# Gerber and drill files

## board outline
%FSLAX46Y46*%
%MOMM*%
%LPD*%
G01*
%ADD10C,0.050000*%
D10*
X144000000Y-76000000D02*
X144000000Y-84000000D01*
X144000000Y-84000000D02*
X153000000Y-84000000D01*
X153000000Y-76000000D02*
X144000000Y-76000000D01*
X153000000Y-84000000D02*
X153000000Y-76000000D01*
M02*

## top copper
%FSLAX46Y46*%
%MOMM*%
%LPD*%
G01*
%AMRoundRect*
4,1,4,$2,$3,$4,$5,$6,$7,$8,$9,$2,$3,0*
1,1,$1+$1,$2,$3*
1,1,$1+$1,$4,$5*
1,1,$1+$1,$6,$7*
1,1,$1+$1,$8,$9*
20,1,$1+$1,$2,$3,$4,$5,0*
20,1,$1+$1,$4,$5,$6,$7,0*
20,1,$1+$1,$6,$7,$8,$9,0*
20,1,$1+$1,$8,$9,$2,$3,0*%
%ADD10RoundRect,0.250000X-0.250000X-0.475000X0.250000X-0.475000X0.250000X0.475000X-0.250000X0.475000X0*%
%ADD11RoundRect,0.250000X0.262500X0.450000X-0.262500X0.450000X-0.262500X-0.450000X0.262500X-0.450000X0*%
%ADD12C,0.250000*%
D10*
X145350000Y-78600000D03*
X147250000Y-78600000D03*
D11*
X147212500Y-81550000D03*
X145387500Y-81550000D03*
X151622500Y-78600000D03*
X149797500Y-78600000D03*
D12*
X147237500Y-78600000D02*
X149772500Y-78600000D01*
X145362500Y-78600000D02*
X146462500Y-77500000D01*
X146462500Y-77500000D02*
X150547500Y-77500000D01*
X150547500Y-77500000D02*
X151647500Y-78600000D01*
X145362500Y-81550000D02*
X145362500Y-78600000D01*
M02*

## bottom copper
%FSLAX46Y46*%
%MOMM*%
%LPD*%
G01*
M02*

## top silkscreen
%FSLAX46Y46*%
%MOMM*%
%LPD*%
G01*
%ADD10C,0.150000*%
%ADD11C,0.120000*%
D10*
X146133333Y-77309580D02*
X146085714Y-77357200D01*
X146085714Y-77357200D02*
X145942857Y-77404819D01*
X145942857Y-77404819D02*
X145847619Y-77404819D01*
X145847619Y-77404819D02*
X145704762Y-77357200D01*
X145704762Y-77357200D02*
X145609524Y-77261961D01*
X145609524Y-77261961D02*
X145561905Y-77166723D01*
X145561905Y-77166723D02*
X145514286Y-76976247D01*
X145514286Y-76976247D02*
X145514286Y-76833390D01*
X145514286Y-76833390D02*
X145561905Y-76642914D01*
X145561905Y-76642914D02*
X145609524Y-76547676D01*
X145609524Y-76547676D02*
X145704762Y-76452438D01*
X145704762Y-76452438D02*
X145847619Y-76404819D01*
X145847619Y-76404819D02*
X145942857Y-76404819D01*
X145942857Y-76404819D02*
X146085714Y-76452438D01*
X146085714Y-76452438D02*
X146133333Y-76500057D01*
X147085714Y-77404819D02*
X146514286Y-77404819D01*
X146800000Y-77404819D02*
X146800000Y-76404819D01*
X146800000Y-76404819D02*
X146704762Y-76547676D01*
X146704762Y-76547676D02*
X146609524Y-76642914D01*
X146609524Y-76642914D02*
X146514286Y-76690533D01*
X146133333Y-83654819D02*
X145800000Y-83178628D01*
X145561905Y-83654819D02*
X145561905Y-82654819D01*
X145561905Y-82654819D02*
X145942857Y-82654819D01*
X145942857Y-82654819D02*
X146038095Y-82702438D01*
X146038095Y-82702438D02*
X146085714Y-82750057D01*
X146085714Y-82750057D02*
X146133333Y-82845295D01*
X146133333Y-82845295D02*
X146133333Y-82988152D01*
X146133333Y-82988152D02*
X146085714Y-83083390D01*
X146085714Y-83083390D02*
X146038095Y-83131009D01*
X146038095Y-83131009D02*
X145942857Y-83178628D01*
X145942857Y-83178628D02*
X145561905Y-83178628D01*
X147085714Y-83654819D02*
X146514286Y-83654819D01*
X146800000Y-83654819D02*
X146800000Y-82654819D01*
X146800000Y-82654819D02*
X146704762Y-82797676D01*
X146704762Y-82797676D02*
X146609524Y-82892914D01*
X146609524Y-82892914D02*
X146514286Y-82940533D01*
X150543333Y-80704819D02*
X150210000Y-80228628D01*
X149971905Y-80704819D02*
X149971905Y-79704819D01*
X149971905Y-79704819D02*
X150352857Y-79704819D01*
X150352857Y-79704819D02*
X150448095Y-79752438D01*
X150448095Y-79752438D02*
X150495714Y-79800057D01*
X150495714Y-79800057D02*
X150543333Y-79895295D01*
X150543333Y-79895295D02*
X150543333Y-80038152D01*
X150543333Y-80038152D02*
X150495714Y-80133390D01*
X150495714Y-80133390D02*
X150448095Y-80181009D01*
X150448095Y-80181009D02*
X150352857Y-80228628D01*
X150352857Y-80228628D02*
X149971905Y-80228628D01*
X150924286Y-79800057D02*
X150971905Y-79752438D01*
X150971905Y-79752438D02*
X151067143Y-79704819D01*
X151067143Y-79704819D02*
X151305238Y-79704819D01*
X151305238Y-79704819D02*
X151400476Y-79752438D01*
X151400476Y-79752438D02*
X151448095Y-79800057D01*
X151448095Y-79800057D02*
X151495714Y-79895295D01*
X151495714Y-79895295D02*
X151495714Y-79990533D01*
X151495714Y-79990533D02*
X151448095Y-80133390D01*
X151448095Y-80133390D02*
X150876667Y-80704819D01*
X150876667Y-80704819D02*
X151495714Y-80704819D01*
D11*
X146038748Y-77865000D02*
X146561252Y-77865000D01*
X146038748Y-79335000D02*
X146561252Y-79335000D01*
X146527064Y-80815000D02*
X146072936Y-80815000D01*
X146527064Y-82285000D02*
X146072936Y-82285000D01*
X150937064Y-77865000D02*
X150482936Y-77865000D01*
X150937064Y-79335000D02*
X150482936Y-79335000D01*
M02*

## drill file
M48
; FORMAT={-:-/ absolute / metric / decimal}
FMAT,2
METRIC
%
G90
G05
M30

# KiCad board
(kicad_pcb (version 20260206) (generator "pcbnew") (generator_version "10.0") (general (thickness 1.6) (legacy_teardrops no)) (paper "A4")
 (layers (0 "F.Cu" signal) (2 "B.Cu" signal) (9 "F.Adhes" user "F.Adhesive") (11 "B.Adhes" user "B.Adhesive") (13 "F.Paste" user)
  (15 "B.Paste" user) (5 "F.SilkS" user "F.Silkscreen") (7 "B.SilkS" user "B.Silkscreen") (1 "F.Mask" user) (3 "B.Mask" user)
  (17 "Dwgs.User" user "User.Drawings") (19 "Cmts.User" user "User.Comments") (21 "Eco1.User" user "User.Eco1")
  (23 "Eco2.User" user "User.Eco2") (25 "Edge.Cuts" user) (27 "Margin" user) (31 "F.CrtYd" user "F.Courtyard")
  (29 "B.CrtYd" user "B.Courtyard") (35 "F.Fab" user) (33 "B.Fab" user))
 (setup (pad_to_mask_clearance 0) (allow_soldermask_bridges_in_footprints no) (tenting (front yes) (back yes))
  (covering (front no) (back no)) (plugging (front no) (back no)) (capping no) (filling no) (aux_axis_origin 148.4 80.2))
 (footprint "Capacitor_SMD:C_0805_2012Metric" (layer "F.Cu") (at 146.3 78.6)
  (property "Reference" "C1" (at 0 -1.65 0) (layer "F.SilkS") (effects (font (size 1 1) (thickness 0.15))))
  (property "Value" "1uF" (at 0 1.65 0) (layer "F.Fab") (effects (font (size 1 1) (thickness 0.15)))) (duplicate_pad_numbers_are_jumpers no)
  (fp_line (start -0.261252 -0.735) (end 0.261252 -0.735) (stroke (width 0.12) (type solid)) (layer "F.SilkS"))
  (fp_line (start -0.261252 0.735) (end 0.261252 0.735) (stroke (width 0.12) (type solid)) (layer "F.SilkS"))
  (pad "1" smd roundrect (at -0.95 0) (size 1 1.45) (layers "F.Cu" "F.Mask" "F.Paste") (roundrect_rratio 0.25) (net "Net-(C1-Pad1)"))
  (pad "2" smd roundrect (at 0.95 0) (size 1 1.45) (layers "F.Cu" "F.Mask" "F.Paste") (roundrect_rratio 0.25) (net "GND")))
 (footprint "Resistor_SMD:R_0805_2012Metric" (layer "F.Cu") (at 146.3 81.55 180)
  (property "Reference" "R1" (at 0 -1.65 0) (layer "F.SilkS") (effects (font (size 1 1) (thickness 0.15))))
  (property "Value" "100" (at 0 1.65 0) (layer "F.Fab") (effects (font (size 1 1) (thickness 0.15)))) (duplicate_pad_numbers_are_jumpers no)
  (fp_line (start -0.227064 0.735) (end 0.227064 0.735) (stroke (width 0.12) (type solid)) (layer "F.SilkS"))
  (fp_line (start -0.227064 -0.735) (end 0.227064 -0.735) (stroke (width 0.12) (type solid)) (layer "F.SilkS"))
  (pad "1" smd roundrect (at -0.9125 0 180) (size 1.025 1.4) (layers "F.Cu" "F.Mask" "F.Paste") (roundrect_rratio 0.243902) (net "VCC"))
  (pad "2" smd roundrect (at 0.9125 0 180) (size 1.025 1.4) (layers "F.Cu" "F.Mask" "F.Paste") (roundrect_rratio 0.243902)
   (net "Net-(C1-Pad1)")))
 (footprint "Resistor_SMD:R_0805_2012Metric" (layer "F.Cu") (at 150.71 78.6 180)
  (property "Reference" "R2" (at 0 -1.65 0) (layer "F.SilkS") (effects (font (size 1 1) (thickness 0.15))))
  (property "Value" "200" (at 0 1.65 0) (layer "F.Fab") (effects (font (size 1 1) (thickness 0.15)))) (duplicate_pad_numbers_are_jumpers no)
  (fp_line (start -0.227064 0.735) (end 0.227064 0.735) (stroke (width 0.12) (type solid)) (layer "F.SilkS"))
  (fp_line (start -0.227064 -0.735) (end 0.227064 -0.735) (stroke (width 0.12) (type solid)) (layer "F.SilkS"))
  (pad "1" smd roundrect (at -0.9125 0 180) (size 1.025 1.4) (layers "F.Cu" "F.Mask" "F.Paste") (roundrect_rratio 0.243902)
   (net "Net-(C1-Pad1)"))
  (pad "2" smd roundrect (at 0.9125 0 180) (size 1.025 1.4) (layers "F.Cu" "F.Mask" "F.Paste") (roundrect_rratio 0.243902) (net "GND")))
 (gr_line (start 144 76) (end 144 84) (stroke (width 0.05) (type solid)) (layer "Edge.Cuts"))
 (gr_line (start 144 84) (end 153 84) (stroke (width 0.05) (type solid)) (layer "Edge.Cuts"))
 (gr_line (start 153 76) (end 144 76) (stroke (width 0.05) (type solid)) (layer "Edge.Cuts"))
 (gr_line (start 153 84) (end 153 76) (stroke (width 0.05) (type solid)) (layer "Edge.Cuts"))
 (segment (start 147.2375 78.6) (end 149.7725 78.6) (width 0.25) (layer "F.Cu") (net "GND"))
 (segment (start 145.3625 78.6) (end 146.4625 77.5) (width 0.25) (layer "F.Cu") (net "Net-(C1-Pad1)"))
 (segment (start 146.4625 77.5) (end 150.5475 77.5) (width 0.25) (layer "F.Cu") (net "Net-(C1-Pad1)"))
 (segment (start 150.5475 77.5) (end 151.6475 78.6) (width 0.25) (layer "F.Cu") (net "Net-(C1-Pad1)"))
 (segment (start 145.3625 81.55) (end 145.3625 78.6) (width 0.25) (layer "F.Cu") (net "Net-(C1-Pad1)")))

